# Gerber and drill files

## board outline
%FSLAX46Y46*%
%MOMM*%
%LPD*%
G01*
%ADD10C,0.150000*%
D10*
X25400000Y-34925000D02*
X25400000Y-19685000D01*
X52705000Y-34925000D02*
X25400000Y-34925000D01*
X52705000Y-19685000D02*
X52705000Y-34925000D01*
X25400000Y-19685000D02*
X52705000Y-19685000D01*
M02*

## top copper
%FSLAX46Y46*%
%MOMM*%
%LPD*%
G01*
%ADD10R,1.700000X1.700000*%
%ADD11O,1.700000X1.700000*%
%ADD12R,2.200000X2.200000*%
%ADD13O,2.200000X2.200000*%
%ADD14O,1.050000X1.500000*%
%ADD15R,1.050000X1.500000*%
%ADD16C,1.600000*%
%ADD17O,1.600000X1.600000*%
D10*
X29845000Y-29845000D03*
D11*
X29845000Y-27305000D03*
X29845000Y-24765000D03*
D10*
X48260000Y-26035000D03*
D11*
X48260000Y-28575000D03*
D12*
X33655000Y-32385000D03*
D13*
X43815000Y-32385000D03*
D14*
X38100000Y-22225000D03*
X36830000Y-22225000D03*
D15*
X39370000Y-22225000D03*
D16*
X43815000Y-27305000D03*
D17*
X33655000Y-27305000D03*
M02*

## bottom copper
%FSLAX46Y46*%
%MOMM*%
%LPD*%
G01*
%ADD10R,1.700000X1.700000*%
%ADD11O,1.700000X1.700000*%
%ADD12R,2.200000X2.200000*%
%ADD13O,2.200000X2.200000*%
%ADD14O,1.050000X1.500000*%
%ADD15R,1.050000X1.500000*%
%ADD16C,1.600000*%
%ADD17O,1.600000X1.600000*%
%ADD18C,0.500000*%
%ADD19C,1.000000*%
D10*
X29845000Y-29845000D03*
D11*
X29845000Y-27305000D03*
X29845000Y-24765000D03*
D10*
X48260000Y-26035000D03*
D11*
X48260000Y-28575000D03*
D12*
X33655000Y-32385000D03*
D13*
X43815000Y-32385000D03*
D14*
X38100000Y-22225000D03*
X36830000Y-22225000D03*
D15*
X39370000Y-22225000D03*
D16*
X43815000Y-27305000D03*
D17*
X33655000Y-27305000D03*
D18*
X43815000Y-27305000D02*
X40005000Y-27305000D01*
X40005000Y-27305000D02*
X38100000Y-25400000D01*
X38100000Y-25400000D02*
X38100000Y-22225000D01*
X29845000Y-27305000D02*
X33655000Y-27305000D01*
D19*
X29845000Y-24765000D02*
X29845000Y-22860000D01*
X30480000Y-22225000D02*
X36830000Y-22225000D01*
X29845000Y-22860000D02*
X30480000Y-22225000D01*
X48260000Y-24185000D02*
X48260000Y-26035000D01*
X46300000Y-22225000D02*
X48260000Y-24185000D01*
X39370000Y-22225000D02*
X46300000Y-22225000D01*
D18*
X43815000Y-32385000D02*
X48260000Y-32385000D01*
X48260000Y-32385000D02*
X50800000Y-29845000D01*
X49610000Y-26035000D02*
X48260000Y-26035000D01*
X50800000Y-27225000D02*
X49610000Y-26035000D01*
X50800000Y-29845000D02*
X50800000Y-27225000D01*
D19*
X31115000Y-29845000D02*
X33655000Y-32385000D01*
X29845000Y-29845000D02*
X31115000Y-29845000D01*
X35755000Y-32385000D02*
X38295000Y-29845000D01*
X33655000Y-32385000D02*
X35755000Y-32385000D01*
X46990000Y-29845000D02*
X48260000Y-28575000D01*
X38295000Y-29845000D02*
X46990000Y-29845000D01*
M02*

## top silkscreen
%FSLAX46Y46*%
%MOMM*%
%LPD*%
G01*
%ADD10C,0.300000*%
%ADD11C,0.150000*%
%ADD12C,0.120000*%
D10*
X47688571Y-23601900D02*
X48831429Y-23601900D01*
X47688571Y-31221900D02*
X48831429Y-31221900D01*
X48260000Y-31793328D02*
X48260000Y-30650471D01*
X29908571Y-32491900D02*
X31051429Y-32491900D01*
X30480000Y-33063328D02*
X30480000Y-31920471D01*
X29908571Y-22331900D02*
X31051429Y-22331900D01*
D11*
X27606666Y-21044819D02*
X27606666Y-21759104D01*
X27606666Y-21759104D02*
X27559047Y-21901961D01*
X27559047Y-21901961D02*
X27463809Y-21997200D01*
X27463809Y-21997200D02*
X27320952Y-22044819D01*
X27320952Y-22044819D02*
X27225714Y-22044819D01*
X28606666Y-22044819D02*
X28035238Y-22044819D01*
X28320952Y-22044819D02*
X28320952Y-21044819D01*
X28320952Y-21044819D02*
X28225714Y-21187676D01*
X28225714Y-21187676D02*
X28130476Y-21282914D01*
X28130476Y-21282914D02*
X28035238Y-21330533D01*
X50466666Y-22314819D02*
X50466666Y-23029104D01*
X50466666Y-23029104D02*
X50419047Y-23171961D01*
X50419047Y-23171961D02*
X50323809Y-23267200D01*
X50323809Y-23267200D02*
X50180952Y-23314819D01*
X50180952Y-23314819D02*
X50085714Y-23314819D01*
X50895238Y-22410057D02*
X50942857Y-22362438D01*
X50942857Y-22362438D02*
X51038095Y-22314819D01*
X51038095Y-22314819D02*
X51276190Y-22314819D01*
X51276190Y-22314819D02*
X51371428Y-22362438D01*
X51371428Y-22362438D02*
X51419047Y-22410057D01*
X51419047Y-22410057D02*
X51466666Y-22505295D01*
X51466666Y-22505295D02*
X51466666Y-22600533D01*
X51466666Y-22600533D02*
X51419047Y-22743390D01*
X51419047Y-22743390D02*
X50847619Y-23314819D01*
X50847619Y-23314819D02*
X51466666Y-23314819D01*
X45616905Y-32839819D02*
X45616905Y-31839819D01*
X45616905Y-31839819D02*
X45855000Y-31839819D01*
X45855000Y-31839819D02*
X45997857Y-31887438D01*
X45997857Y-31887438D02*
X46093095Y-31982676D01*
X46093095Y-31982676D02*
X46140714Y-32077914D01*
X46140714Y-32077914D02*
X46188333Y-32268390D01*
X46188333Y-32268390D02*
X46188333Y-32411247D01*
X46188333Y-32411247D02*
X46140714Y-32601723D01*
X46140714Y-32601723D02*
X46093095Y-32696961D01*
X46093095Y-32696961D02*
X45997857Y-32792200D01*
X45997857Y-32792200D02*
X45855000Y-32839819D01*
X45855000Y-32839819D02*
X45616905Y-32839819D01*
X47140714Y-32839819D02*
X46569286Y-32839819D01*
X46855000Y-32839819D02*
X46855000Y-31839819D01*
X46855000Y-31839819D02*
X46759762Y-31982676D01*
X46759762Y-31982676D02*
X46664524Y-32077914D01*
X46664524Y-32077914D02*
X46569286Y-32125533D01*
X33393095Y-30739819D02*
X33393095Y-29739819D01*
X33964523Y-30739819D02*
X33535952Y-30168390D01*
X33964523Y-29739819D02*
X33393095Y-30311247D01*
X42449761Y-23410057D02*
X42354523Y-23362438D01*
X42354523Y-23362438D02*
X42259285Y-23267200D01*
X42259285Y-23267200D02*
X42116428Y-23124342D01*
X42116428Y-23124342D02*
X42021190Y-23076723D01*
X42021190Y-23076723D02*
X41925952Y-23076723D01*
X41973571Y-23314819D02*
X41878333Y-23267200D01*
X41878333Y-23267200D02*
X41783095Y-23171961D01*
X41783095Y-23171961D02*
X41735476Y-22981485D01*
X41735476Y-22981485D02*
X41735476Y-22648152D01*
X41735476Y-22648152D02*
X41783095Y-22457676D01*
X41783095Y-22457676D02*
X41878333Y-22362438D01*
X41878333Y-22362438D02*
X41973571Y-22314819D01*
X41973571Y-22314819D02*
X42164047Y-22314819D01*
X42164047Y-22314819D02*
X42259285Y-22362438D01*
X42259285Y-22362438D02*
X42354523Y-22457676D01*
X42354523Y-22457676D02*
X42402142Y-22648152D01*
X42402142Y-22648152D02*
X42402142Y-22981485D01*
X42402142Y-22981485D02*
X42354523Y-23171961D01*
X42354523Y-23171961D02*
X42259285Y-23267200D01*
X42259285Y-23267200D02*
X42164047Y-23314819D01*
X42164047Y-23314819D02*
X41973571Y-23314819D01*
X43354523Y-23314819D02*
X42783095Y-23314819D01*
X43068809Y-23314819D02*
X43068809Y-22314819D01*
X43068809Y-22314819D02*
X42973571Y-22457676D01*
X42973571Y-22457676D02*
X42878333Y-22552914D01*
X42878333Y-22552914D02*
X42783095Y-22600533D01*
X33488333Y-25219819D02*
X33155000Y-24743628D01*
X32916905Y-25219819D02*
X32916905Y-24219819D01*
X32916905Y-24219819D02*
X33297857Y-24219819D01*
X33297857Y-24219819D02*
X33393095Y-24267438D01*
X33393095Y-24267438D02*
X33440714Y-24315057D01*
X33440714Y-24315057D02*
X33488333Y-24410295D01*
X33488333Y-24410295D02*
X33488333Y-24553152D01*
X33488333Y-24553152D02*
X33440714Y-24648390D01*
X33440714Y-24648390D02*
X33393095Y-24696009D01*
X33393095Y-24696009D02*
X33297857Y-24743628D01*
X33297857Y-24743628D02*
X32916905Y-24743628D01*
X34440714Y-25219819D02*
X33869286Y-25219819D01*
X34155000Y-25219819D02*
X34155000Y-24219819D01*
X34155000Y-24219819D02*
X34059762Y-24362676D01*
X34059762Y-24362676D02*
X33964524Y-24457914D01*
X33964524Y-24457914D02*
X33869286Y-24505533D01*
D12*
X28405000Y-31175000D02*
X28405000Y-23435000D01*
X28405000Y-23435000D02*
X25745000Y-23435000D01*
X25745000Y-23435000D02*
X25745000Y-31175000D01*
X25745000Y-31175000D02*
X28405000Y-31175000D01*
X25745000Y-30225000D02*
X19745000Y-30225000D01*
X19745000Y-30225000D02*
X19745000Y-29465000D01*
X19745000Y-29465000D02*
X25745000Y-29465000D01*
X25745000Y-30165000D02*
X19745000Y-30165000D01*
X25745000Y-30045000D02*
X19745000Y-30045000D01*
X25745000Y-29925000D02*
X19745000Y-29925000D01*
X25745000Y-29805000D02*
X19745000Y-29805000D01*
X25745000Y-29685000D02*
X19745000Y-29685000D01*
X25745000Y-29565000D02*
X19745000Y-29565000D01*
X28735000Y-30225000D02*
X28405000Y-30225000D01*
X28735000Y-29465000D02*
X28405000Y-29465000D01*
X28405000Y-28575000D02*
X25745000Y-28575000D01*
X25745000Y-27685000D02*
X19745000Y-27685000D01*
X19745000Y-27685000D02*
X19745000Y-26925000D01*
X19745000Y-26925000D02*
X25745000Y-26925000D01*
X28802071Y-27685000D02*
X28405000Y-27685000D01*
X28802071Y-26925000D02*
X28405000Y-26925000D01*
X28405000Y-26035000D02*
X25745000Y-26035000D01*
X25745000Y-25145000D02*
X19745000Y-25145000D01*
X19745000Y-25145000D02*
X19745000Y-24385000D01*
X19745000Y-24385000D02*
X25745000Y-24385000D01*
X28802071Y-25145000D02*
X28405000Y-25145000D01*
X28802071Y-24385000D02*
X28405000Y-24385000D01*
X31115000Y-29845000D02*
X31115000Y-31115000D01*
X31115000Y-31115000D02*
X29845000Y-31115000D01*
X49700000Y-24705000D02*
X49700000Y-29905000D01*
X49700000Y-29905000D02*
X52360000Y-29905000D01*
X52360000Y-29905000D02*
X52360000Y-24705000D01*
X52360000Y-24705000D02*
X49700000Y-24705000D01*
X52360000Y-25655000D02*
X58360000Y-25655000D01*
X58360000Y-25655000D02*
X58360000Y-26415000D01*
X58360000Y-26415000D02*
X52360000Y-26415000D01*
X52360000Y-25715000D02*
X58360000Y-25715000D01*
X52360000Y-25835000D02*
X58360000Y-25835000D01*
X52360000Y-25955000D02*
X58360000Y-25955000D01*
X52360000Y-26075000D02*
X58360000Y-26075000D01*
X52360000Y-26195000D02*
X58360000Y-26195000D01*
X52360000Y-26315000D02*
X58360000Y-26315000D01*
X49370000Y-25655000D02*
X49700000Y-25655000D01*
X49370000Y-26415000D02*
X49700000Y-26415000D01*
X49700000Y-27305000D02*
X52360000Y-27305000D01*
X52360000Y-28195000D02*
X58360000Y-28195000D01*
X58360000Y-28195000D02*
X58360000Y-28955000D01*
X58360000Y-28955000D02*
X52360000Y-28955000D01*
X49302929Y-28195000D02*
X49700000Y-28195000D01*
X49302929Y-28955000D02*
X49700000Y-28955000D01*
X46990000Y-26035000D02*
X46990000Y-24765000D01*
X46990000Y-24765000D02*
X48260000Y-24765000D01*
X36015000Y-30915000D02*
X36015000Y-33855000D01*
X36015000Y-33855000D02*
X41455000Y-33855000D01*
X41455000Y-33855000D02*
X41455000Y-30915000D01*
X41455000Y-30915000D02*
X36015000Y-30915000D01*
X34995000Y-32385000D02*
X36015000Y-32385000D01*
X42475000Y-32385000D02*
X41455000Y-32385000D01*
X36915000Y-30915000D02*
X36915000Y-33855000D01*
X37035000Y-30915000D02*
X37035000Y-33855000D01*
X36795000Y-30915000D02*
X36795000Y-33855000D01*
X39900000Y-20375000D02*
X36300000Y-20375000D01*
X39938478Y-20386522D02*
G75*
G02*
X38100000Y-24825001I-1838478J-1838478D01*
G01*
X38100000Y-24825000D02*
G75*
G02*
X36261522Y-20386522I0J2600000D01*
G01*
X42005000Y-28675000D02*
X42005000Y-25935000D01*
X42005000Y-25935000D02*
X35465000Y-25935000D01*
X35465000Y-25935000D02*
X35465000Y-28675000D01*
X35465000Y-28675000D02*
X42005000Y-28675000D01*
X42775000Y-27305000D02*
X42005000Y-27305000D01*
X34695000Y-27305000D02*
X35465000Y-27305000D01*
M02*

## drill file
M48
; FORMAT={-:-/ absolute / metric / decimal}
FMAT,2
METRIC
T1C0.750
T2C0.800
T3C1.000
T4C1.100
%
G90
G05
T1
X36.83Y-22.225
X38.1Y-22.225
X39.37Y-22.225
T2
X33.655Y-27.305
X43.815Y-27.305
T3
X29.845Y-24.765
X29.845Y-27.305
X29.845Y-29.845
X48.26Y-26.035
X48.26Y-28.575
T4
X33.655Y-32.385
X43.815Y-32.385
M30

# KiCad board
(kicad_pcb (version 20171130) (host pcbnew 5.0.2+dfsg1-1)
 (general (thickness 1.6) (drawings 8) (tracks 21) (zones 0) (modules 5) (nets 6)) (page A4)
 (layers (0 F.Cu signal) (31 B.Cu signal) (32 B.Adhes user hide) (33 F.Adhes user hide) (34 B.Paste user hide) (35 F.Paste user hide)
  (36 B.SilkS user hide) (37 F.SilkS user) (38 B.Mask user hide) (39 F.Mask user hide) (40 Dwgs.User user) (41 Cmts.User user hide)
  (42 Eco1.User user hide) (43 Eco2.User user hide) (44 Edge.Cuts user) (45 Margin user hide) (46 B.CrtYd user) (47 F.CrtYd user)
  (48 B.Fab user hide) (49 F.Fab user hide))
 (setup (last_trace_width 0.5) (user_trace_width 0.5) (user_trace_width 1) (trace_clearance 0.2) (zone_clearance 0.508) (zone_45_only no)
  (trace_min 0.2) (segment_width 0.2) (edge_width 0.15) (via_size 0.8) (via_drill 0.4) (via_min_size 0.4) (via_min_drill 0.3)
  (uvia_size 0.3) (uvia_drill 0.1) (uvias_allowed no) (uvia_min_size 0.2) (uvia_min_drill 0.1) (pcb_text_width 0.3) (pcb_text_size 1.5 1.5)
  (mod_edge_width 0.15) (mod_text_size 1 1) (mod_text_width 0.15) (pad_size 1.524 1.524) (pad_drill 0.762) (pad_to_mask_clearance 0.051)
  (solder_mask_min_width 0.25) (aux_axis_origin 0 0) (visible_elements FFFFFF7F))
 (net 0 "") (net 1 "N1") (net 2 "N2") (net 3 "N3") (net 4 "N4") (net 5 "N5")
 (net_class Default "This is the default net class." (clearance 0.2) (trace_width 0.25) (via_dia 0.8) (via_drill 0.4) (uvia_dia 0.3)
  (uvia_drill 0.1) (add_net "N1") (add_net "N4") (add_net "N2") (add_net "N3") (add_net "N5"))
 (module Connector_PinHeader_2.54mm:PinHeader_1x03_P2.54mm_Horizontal (layer F.Cu) (at 29.845 29.845 180)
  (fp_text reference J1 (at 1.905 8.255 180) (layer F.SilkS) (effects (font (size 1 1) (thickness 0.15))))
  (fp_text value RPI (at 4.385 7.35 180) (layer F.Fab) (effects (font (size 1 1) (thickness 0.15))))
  (fp_line (start 1.44 -1.33) (end 1.44 6.41) (layer F.SilkS) (width 0.12))
  (fp_line (start 1.44 6.41) (end 4.1 6.41) (layer F.SilkS) (width 0.12))
  (fp_line (start 4.1 6.41) (end 4.1 -1.33) (layer F.SilkS) (width 0.12))
  (fp_line (start 4.1 -1.33) (end 1.44 -1.33) (layer F.SilkS) (width 0.12))
  (fp_line (start 4.1 -0.38) (end 10.1 -0.38) (layer F.SilkS) (width 0.12))
  (fp_line (start 10.1 -0.38) (end 10.1 0.38) (layer F.SilkS) (width 0.12))
  (fp_line (start 10.1 0.38) (end 4.1 0.38) (layer F.SilkS) (width 0.12))
  (fp_line (start 4.1 -0.32) (end 10.1 -0.32) (layer F.SilkS) (width 0.12))
  (fp_line (start 4.1 -0.2) (end 10.1 -0.2) (layer F.SilkS) (width 0.12))
  (fp_line (start 4.1 -0.08) (end 10.1 -0.08) (layer F.SilkS) (width 0.12))
  (fp_line (start 4.1 0.04) (end 10.1 0.04) (layer F.SilkS) (width 0.12))
  (fp_line (start 4.1 0.16) (end 10.1 0.16) (layer F.SilkS) (width 0.12))
  (fp_line (start 4.1 0.28) (end 10.1 0.28) (layer F.SilkS) (width 0.12))
  (fp_line (start 1.11 -0.38) (end 1.44 -0.38) (layer F.SilkS) (width 0.12))
  (fp_line (start 1.11 0.38) (end 1.44 0.38) (layer F.SilkS) (width 0.12))
  (fp_line (start 1.44 1.27) (end 4.1 1.27) (layer F.SilkS) (width 0.12))
  (fp_line (start 4.1 2.16) (end 10.1 2.16) (layer F.SilkS) (width 0.12))
  (fp_line (start 10.1 2.16) (end 10.1 2.92) (layer F.SilkS) (width 0.12))
  (fp_line (start 10.1 2.92) (end 4.1 2.92) (layer F.SilkS) (width 0.12))
  (fp_line (start 1.042929 2.16) (end 1.44 2.16) (layer F.SilkS) (width 0.12))
  (fp_line (start 1.042929 2.92) (end 1.44 2.92) (layer F.SilkS) (width 0.12))
  (fp_line (start 1.44 3.81) (end 4.1 3.81) (layer F.SilkS) (width 0.12))
  (fp_line (start 4.1 4.7) (end 10.1 4.7) (layer F.SilkS) (width 0.12))
  (fp_line (start 10.1 4.7) (end 10.1 5.46) (layer F.SilkS) (width 0.12))
  (fp_line (start 10.1 5.46) (end 4.1 5.46) (layer F.SilkS) (width 0.12))
  (fp_line (start 1.042929 4.7) (end 1.44 4.7) (layer F.SilkS) (width 0.12))
  (fp_line (start 1.042929 5.46) (end 1.44 5.46) (layer F.SilkS) (width 0.12))
  (fp_line (start -1.27 0) (end -1.27 -1.27) (layer F.SilkS) (width 0.12))
  (fp_line (start -1.27 -1.27) (end 0 -1.27) (layer F.SilkS) (width 0.12))
  (pad 1 thru_hole rect (at 0 0 180) (size 1.7 1.7) (drill 1) (layers *.Cu *.Mask) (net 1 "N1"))
  (pad 2 thru_hole oval (at 0 2.54 180) (size 1.7 1.7) (drill 1) (layers *.Cu *.Mask) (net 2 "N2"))
  (pad 3 thru_hole oval (at 0 5.08 180) (size 1.7 1.7) (drill 1) (layers *.Cu *.Mask) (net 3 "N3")))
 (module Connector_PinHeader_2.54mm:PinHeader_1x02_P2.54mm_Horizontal (layer F.Cu) (at 48.26 26.035)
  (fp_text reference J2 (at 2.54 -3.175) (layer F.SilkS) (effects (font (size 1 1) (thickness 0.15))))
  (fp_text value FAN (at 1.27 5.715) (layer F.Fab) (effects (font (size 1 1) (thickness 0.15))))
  (fp_line (start 1.44 -1.33) (end 1.44 3.87) (layer F.SilkS) (width 0.12))
  (fp_line (start 1.44 3.87) (end 4.1 3.87) (layer F.SilkS) (width 0.12))
  (fp_line (start 4.1 3.87) (end 4.1 -1.33) (layer F.SilkS) (width 0.12))
  (fp_line (start 4.1 -1.33) (end 1.44 -1.33) (layer F.SilkS) (width 0.12))
  (fp_line (start 4.1 -0.38) (end 10.1 -0.38) (layer F.SilkS) (width 0.12))
  (fp_line (start 10.1 -0.38) (end 10.1 0.38) (layer F.SilkS) (width 0.12))
  (fp_line (start 10.1 0.38) (end 4.1 0.38) (layer F.SilkS) (width 0.12))
  (fp_line (start 4.1 -0.32) (end 10.1 -0.32) (layer F.SilkS) (width 0.12))
  (fp_line (start 4.1 -0.2) (end 10.1 -0.2) (layer F.SilkS) (width 0.12))
  (fp_line (start 4.1 -0.08) (end 10.1 -0.08) (layer F.SilkS) (width 0.12))
  (fp_line (start 4.1 0.04) (end 10.1 0.04) (layer F.SilkS) (width 0.12))
  (fp_line (start 4.1 0.16) (end 10.1 0.16) (layer F.SilkS) (width 0.12))
  (fp_line (start 4.1 0.28) (end 10.1 0.28) (layer F.SilkS) (width 0.12))
  (fp_line (start 1.11 -0.38) (end 1.44 -0.38) (layer F.SilkS) (width 0.12))
  (fp_line (start 1.11 0.38) (end 1.44 0.38) (layer F.SilkS) (width 0.12))
  (fp_line (start 1.44 1.27) (end 4.1 1.27) (layer F.SilkS) (width 0.12))
  (fp_line (start 4.1 2.16) (end 10.1 2.16) (layer F.SilkS) (width 0.12))
  (fp_line (start 10.1 2.16) (end 10.1 2.92) (layer F.SilkS) (width 0.12))
  (fp_line (start 10.1 2.92) (end 4.1 2.92) (layer F.SilkS) (width 0.12))
  (fp_line (start 1.042929 2.16) (end 1.44 2.16) (layer F.SilkS) (width 0.12))
  (fp_line (start 1.042929 2.92) (end 1.44 2.92) (layer F.SilkS) (width 0.12))
  (fp_line (start -1.27 0) (end -1.27 -1.27) (layer F.SilkS) (width 0.12))
  (fp_line (start -1.27 -1.27) (end 0 -1.27) (layer F.SilkS) (width 0.12))
  (pad 1 thru_hole rect (at 0 0) (size 1.7 1.7) (drill 1) (layers *.Cu *.Mask) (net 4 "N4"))
  (pad 2 thru_hole oval (at 0 2.54) (size 1.7 1.7) (drill 1) (layers *.Cu *.Mask) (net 1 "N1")))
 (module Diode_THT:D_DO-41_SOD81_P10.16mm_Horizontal (layer F.Cu) (at 33.655 32.385)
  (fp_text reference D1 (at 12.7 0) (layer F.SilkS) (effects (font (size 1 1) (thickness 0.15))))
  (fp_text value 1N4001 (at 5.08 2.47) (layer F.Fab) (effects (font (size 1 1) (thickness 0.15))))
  (fp_line (start 2.36 -1.47) (end 2.36 1.47) (layer F.SilkS) (width 0.12))
  (fp_line (start 2.36 1.47) (end 7.8 1.47) (layer F.SilkS) (width 0.12))
  (fp_line (start 7.8 1.47) (end 7.8 -1.47) (layer F.SilkS) (width 0.12))
  (fp_line (start 7.8 -1.47) (end 2.36 -1.47) (layer F.SilkS) (width 0.12))
  (fp_line (start 1.34 0) (end 2.36 0) (layer F.SilkS) (width 0.12))
  (fp_line (start 8.82 0) (end 7.8 0) (layer F.SilkS) (width 0.12))
  (fp_line (start 3.26 -1.47) (end 3.26 1.47) (layer F.SilkS) (width 0.12))
  (fp_line (start 3.38 -1.47) (end 3.38 1.47) (layer F.SilkS) (width 0.12))
  (fp_line (start 3.14 -1.47) (end 3.14 1.47) (layer F.SilkS) (width 0.12))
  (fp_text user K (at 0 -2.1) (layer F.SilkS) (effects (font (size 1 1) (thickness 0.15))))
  (pad 1 thru_hole rect (at 0 0) (size 2.2 2.2) (drill 1.1) (layers *.Cu *.Mask) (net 1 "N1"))
  (pad 2 thru_hole oval (at 10.16 0) (size 2.2 2.2) (drill 1.1) (layers *.Cu *.Mask) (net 4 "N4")))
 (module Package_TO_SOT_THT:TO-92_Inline (layer F.Cu) (at 39.37 22.225 180)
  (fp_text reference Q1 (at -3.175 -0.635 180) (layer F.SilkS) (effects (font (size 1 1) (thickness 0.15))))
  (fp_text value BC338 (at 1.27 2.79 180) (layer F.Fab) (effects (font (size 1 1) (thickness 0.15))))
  (fp_line (start -0.53 1.85) (end 3.07 1.85) (layer F.SilkS) (width 0.12))
  (fp_arc (start 1.27 0) (end 1.27 -2.6) (angle -135) (layer F.SilkS) (width 0.12))
  (fp_arc (start 1.27 0) (end 1.27 -2.6) (angle 135) (layer F.SilkS) (width 0.12))
  (pad 2 thru_hole oval (at 1.27 0 180) (size 1.05 1.5) (drill 0.75) (layers *.Cu *.Mask) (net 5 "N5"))
  (pad 3 thru_hole oval (at 2.54 0 180) (size 1.05 1.5) (drill 0.75) (layers *.Cu *.Mask) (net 3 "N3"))
  (pad 1 thru_hole rect (at 0 0 180) (size 1.05 1.5) (drill 0.75) (layers *.Cu *.Mask) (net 4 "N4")))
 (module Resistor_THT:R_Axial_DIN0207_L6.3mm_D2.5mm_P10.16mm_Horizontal (layer F.Cu) (at 43.815 27.305 180)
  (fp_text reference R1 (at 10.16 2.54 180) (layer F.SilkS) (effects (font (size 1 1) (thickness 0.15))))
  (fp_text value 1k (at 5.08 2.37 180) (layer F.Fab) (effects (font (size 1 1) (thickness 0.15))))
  (fp_line (start 1.81 -1.37) (end 1.81 1.37) (layer F.SilkS) (width 0.12))
  (fp_line (start 1.81 1.37) (end 8.35 1.37) (layer F.SilkS) (width 0.12))
  (fp_line (start 8.35 1.37) (end 8.35 -1.37) (layer F.SilkS) (width 0.12))
  (fp_line (start 8.35 -1.37) (end 1.81 -1.37) (layer F.SilkS) (width 0.12))
  (fp_line (start 1.04 0) (end 1.81 0) (layer F.SilkS) (width 0.12))
  (fp_line (start 9.12 0) (end 8.35 0) (layer F.SilkS) (width 0.12))
  (pad 1 thru_hole circle (at 0 0 180) (size 1.6 1.6) (drill 0.8) (layers *.Cu *.Mask) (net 5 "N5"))
  (pad 2 thru_hole oval (at 10.16 0 180) (size 1.6 1.6) (drill 0.8) (layers *.Cu *.Mask) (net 2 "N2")))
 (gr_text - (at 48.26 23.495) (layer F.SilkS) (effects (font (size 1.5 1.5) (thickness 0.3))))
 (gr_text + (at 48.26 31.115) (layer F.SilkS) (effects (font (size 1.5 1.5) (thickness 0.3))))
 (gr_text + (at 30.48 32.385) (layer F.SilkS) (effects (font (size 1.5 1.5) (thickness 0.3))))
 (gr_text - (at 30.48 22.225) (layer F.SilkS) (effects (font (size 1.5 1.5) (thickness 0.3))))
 (gr_line (start 25.4 34.925) (end 25.4 19.685) (layer Edge.Cuts) (width 0.15))
 (gr_line (start 52.705 34.925) (end 25.4 34.925) (layer Edge.Cuts) (width 0.15))
 (gr_line (start 52.705 19.685) (end 52.705 34.925) (layer Edge.Cuts) (width 0.15))
 (gr_line (start 25.4 19.685) (end 52.705 19.685) (layer Edge.Cuts) (width 0.15))
 (segment (start 43.815 27.305) (end 40.005 27.305) (width 0.5) (layer B.Cu) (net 5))
 (segment (start 40.005 27.305) (end 38.1 25.4) (width 0.5) (layer B.Cu) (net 5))
 (segment (start 38.1 25.4) (end 38.1 22.225) (width 0.5) (layer B.Cu) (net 5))
 (segment (start 29.845 27.305) (end 33.655 27.305) (width 0.5) (layer B.Cu) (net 2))
 (segment (start 29.845 24.765) (end 29.845 22.86) (width 1) (layer B.Cu) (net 3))
 (segment (start 30.48 22.225) (end 36.83 22.225) (width 1) (layer B.Cu) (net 3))
 (segment (start 29.845 22.86) (end 30.48 22.225) (width 1) (layer B.Cu) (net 3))
 (segment (start 48.26 24.185) (end 48.26 26.035) (width 1) (layer B.Cu) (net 4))
 (segment (start 46.3 22.225) (end 48.26 24.185) (width 1) (layer B.Cu) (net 4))
 (segment (start 39.37 22.225) (end 46.3 22.225) (width 1) (layer B.Cu) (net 4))
 (segment (start 43.815 32.385) (end 48.26 32.385) (width 0.5) (layer B.Cu) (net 4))
 (segment (start 48.26 32.385) (end 50.8 29.845) (width 0.5) (layer B.Cu) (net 4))
 (segment (start 49.61 26.035) (end 48.26 26.035) (width 0.5) (layer B.Cu) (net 4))
 (segment (start 50.8 27.225) (end 49.61 26.035) (width 0.5) (layer B.Cu) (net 4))
 (segment (start 50.8 29.845) (end 50.8 27.225) (width 0.5) (layer B.Cu) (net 4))
 (segment (start 31.115 29.845) (end 33.655 32.385) (width 1) (layer B.Cu) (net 1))
 (segment (start 29.845 29.845) (end 31.115 29.845) (width 1) (layer B.Cu) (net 1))
 (segment (start 35.755 32.385) (end 38.295 29.845) (width 1) (layer B.Cu) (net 1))
 (segment (start 33.655 32.385) (end 35.755 32.385) (width 1) (layer B.Cu) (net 1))
 (segment (start 46.99 29.845) (end 48.26 28.575) (width 1) (layer B.Cu) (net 1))
 (segment (start 38.295 29.845) (end 46.99 29.845) (width 1) (layer B.Cu) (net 1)))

